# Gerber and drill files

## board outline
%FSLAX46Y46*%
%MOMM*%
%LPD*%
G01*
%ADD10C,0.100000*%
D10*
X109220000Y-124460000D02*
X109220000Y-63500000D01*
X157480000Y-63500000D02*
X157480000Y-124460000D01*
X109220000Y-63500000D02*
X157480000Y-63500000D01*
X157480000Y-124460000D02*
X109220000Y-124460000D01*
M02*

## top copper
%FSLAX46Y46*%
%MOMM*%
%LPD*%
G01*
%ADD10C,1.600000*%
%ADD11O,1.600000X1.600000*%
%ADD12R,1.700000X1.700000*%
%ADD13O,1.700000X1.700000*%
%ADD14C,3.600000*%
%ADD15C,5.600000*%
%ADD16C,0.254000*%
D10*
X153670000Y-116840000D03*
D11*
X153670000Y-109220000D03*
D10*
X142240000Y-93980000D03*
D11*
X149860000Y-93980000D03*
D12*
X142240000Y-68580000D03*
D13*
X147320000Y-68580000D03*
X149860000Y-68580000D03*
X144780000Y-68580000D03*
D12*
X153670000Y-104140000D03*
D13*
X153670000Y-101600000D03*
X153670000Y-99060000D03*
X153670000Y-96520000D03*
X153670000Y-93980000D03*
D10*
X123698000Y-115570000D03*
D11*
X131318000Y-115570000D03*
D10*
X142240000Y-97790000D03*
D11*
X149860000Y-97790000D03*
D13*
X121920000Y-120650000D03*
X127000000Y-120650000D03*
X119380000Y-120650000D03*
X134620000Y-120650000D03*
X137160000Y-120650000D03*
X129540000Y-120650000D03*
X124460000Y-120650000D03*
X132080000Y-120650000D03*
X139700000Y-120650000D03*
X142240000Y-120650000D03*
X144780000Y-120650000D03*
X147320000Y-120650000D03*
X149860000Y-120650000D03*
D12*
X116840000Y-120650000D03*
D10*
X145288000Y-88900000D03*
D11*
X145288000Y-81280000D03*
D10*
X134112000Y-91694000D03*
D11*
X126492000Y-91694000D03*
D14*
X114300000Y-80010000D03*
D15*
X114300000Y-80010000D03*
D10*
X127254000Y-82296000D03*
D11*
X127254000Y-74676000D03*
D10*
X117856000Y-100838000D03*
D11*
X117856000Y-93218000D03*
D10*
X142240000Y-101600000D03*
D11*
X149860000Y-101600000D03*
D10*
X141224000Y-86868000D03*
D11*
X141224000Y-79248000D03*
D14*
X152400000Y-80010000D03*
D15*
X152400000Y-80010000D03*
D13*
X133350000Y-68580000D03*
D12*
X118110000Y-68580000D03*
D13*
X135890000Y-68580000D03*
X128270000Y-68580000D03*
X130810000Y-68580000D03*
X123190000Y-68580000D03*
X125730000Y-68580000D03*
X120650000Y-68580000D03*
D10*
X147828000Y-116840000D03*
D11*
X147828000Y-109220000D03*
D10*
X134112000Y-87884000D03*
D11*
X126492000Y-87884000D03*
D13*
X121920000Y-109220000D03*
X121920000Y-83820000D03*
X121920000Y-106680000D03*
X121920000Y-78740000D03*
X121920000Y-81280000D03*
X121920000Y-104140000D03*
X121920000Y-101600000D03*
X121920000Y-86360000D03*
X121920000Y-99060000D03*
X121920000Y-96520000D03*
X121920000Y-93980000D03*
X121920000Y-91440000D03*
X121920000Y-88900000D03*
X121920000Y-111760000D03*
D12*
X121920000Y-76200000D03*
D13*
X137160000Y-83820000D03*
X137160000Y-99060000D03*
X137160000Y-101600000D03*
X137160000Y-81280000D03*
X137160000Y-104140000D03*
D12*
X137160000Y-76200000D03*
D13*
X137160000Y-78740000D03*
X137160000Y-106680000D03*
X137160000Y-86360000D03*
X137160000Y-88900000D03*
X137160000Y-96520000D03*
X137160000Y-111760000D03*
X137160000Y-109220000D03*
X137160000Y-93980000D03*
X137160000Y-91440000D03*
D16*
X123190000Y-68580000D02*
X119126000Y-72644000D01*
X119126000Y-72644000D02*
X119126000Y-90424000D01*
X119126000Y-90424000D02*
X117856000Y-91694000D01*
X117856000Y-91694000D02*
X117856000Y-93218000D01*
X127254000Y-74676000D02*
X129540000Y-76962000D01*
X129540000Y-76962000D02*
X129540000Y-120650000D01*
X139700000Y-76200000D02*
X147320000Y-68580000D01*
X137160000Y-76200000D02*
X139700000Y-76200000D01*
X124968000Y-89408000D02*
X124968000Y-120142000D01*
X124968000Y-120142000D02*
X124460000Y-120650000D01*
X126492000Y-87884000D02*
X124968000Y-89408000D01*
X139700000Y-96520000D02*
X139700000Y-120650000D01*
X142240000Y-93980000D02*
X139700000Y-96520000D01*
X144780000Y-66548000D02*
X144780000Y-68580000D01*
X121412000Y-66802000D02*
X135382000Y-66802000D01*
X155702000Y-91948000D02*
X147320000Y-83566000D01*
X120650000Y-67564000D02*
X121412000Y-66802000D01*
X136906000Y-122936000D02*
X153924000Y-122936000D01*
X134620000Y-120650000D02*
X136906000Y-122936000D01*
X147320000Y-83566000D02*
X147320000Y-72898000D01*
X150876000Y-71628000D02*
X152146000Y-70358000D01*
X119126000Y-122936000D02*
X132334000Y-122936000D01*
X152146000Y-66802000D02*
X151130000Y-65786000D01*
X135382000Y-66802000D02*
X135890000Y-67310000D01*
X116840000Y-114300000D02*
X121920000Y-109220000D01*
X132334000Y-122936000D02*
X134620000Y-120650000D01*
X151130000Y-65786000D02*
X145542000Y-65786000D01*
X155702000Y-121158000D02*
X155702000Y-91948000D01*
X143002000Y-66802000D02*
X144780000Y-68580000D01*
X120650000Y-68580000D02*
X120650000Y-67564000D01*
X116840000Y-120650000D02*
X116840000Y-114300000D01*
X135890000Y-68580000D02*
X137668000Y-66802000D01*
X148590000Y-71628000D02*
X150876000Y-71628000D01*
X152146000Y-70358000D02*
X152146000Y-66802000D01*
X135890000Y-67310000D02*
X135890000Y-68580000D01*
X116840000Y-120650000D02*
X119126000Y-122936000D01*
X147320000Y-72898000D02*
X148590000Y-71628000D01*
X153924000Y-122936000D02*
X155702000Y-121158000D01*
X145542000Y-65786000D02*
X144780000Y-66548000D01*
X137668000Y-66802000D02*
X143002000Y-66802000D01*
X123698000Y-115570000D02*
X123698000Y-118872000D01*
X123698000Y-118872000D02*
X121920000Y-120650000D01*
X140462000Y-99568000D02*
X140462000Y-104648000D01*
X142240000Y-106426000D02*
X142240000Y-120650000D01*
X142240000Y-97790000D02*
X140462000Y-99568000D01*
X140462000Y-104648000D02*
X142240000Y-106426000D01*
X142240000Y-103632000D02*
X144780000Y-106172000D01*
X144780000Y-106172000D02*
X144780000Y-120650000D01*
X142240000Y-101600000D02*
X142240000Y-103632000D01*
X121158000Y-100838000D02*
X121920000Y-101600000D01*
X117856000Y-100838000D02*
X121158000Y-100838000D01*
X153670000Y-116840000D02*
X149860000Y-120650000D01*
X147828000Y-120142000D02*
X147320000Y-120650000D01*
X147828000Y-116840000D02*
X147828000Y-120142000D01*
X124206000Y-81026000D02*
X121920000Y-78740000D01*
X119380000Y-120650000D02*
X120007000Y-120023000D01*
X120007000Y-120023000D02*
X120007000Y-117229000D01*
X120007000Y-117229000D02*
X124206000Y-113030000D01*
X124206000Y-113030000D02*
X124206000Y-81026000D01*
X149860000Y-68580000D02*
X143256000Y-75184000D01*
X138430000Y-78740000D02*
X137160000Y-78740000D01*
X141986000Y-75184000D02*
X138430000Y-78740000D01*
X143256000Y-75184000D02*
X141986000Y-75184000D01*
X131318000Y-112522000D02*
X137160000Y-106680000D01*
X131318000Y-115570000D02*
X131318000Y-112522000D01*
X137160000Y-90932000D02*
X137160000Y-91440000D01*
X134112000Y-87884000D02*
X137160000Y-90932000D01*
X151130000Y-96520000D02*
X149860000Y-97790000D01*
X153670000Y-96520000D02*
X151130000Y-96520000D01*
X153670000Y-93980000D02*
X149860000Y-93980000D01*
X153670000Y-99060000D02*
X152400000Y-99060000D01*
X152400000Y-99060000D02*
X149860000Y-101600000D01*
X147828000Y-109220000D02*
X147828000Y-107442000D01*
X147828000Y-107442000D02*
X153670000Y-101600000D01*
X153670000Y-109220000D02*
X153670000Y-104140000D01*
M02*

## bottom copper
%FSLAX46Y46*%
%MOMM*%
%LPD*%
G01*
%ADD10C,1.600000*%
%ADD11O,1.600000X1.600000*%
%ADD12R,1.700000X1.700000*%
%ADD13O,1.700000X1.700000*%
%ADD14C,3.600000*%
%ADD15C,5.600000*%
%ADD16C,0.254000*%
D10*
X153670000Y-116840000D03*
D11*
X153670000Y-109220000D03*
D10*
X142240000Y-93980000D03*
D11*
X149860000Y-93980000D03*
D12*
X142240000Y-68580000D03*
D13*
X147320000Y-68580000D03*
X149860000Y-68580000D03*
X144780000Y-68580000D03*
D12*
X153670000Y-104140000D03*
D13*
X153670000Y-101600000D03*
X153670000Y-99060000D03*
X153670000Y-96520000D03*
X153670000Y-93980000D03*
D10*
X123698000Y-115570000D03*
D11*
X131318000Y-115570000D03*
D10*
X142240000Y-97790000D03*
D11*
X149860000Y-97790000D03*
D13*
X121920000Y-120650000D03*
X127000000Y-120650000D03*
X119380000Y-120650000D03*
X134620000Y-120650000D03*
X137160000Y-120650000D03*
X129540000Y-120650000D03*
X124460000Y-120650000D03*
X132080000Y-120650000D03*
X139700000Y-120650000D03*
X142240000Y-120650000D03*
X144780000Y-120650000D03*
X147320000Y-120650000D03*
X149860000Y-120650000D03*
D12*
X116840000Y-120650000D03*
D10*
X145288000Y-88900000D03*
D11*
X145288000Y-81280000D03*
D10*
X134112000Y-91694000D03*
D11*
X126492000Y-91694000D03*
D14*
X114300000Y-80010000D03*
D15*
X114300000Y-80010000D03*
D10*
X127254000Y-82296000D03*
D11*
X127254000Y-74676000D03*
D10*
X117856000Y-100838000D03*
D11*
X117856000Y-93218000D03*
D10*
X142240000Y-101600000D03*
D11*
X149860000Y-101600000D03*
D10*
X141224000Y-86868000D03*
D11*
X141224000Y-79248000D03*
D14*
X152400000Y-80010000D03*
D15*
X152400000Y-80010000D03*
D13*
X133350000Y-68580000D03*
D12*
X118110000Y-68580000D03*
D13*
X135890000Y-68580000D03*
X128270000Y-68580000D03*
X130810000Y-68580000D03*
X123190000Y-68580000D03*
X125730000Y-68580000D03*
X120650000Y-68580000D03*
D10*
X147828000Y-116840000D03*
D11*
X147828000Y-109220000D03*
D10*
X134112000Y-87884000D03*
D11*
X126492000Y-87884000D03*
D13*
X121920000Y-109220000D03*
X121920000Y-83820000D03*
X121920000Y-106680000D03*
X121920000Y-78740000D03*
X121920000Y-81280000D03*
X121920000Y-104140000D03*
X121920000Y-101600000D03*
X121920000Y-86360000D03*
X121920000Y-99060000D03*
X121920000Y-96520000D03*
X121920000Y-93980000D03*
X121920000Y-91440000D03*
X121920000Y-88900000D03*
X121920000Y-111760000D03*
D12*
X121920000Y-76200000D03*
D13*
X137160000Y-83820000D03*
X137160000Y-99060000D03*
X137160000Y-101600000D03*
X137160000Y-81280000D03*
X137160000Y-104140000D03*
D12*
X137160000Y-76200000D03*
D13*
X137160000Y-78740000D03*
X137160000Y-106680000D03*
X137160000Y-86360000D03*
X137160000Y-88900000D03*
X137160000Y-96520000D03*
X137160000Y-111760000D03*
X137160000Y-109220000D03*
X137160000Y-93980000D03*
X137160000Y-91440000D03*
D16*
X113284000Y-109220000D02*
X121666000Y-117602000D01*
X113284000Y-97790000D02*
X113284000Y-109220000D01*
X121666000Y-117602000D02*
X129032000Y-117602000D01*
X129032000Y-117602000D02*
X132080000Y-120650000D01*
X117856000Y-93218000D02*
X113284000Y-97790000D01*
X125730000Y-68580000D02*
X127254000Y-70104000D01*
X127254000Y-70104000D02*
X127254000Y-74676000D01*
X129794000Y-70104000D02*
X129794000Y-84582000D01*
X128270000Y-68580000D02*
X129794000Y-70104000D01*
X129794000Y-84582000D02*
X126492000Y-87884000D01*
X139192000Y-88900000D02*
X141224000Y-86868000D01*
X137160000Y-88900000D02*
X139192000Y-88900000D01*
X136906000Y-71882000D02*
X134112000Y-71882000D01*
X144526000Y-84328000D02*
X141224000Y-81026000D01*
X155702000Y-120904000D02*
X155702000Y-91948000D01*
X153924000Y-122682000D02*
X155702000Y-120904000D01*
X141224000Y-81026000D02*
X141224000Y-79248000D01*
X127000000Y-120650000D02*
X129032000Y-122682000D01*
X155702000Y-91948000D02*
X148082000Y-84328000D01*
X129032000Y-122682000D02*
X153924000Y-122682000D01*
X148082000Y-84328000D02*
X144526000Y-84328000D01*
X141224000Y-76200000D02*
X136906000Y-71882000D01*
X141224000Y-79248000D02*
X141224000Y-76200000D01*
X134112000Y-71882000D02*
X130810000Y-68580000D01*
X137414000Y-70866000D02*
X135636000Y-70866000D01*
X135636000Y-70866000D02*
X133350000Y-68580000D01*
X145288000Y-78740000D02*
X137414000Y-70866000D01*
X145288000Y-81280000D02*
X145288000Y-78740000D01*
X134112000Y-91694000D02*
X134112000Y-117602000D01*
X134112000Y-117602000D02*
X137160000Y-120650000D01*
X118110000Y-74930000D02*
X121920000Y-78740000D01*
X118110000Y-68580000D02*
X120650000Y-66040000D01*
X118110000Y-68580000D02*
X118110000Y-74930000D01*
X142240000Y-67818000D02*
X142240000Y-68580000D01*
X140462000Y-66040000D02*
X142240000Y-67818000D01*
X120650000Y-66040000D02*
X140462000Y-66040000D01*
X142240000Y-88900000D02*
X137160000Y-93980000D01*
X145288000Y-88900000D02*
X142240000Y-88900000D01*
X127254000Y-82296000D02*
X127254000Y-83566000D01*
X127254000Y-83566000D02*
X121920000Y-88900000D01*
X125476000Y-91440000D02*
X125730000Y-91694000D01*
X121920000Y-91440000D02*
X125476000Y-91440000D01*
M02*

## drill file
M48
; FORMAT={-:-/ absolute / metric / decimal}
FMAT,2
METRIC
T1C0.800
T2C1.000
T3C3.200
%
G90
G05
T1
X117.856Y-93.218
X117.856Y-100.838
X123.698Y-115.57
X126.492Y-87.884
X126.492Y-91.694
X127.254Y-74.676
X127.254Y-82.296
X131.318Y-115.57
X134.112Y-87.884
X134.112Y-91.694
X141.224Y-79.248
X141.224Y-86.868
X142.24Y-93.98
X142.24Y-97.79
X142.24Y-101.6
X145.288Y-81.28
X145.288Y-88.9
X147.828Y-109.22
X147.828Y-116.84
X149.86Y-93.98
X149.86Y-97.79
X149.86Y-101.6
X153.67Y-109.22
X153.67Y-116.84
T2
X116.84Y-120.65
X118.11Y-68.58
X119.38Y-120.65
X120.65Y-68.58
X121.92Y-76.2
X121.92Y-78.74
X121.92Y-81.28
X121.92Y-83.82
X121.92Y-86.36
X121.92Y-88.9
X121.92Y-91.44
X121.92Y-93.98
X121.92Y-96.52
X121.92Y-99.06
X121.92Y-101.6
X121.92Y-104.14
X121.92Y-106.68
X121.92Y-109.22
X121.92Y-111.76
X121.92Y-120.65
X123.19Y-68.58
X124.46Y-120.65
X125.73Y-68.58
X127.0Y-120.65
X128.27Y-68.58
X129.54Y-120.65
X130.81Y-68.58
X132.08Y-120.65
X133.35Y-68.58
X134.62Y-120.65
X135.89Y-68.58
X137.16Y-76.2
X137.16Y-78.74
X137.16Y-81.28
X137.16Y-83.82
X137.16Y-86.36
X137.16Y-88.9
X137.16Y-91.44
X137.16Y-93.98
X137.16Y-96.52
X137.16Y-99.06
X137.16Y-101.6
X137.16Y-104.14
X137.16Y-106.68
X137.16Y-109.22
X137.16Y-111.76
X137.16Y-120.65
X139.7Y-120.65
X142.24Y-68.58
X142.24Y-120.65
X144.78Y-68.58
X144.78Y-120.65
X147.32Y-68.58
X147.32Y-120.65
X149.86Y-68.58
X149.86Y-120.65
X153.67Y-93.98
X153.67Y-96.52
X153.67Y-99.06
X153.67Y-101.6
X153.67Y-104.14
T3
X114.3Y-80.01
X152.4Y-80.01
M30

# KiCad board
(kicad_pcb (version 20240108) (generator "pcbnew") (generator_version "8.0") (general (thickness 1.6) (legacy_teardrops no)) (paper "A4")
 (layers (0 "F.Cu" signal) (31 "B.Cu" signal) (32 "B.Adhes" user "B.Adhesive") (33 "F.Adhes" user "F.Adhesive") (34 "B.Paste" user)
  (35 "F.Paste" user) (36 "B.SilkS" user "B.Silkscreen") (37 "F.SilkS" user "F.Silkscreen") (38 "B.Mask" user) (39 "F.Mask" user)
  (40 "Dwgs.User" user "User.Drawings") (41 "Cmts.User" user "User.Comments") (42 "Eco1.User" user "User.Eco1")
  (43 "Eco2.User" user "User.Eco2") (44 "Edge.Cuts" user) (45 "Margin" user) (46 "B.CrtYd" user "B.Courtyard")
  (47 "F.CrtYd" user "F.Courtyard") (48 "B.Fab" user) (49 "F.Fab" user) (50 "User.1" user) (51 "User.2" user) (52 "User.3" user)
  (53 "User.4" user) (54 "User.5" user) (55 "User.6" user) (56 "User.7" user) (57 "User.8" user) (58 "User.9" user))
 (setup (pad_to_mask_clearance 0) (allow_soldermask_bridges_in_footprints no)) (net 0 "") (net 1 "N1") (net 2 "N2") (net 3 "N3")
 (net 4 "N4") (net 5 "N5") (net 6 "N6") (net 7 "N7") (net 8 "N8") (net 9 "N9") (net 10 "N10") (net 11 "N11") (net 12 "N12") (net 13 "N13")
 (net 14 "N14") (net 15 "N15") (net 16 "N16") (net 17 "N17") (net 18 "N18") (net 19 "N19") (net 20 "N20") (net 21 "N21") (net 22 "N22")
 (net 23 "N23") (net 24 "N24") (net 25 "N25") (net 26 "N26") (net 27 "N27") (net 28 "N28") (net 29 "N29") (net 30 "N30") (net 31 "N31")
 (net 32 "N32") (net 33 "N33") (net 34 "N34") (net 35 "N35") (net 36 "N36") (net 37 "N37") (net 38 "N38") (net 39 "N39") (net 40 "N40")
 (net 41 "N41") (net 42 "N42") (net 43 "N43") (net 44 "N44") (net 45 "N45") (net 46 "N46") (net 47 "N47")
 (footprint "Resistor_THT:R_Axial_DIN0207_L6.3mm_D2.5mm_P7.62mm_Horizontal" (layer "F.Cu") (at 153.67 116.84 90)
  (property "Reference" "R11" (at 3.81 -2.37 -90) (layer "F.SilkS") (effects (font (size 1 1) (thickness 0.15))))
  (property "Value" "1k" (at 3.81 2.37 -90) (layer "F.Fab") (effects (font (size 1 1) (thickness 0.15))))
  (pad "1" thru_hole circle (at 0 0 90) (size 1.6 1.6) (drill 0.8) (layers "*.Cu" "*.Mask") (remove_unused_layers no) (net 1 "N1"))
  (pad "2" thru_hole oval (at 7.62 0 90) (size 1.6 1.6) (drill 0.8) (layers "*.Cu" "*.Mask") (remove_unused_layers no) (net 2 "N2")))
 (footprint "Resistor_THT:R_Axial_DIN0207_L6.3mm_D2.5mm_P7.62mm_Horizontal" (layer "F.Cu") (at 142.24 93.98)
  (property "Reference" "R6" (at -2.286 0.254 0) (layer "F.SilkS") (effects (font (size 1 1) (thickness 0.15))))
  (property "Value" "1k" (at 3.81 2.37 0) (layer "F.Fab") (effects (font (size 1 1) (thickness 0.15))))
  (pad "1" thru_hole circle (at 0 0) (size 1.6 1.6) (drill 0.8) (layers "*.Cu" "*.Mask") (remove_unused_layers no) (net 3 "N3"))
  (pad "2" thru_hole oval (at 7.62 0) (size 1.6 1.6) (drill 0.8) (layers "*.Cu" "*.Mask") (remove_unused_layers no) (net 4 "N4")))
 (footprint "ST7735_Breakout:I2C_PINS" (layer "F.Cu") (at 142.24 68.58 90)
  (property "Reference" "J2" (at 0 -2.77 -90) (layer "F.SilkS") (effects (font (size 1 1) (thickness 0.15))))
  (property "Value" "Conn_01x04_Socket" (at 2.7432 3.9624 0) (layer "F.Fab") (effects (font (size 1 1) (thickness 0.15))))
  (pad "GND" thru_hole rect (at 0 0 180) (size 1.7 1.7) (drill 1) (layers "*.Cu" "*.Mask") (remove_unused_layers no) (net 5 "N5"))
  (pad "SCK" thru_hole oval (at 0 5.08 90) (size 1.7 1.7) (drill 1) (layers "*.Cu" "*.Mask") (remove_unused_layers no) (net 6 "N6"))
  (pad "SDA" thru_hole oval (at 0 7.62 90) (size 1.7 1.7) (drill 1) (layers "*.Cu" "*.Mask") (remove_unused_layers no) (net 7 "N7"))
  (pad "VCC" thru_hole oval (at 0 2.54 90) (size 1.7 1.7) (drill 1) (layers "*.Cu" "*.Mask") (remove_unused_layers no) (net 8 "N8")))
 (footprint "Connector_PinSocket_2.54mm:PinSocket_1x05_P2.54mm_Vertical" (layer "F.Cu") (at 153.67 104.14 180)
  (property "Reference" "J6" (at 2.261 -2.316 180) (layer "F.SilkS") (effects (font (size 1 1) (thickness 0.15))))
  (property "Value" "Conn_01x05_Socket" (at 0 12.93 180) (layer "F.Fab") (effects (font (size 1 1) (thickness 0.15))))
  (pad "1" thru_hole rect (at 0 0 180) (size 1.7 1.7) (drill 1) (layers "*.Cu" "*.Mask") (remove_unused_layers no) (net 2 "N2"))
  (pad "2" thru_hole oval (at 0 2.54 180) (size 1.7 1.7) (drill 1) (layers "*.Cu" "*.Mask") (remove_unused_layers no) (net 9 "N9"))
  (pad "3" thru_hole oval (at 0 5.08 180) (size 1.7 1.7) (drill 1) (layers "*.Cu" "*.Mask") (remove_unused_layers no) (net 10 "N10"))
  (pad "4" thru_hole oval (at 0 7.62 180) (size 1.7 1.7) (drill 1) (layers "*.Cu" "*.Mask") (remove_unused_layers no) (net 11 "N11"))
  (pad "5" thru_hole oval (at 0 10.16 180) (size 1.7 1.7) (drill 1) (layers "*.Cu" "*.Mask") (remove_unused_layers no) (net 4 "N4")))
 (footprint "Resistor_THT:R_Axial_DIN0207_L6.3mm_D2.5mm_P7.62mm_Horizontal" (layer "F.Cu") (at 123.698 115.57)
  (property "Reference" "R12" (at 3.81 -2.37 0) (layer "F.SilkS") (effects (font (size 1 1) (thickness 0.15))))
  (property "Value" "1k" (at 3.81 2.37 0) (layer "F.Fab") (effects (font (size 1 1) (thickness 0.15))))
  (pad "1" thru_hole circle (at 0 0) (size 1.6 1.6) (drill 0.8) (layers "*.Cu" "*.Mask") (remove_unused_layers no) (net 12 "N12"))
  (pad "2" thru_hole oval (at 7.62 0) (size 1.6 1.6) (drill 0.8) (layers "*.Cu" "*.Mask") (remove_unused_layers no) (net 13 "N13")))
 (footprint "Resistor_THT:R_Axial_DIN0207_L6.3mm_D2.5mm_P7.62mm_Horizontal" (layer "F.Cu") (at 142.24 97.79)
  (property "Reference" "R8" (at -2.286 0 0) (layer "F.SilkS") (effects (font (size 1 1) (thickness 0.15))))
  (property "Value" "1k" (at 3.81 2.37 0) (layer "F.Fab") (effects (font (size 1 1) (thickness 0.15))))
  (pad "1" thru_hole circle (at 0 0) (size 1.6 1.6) (drill 0.8) (layers "*.Cu" "*.Mask") (remove_unused_layers no) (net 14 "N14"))
  (pad "2" thru_hole oval (at 7.62 0) (size 1.6 1.6) (drill 0.8) (layers "*.Cu" "*.Mask") (remove_unused_layers no) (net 11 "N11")))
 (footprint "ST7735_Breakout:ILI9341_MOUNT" (layer "F.Cu") (at 116.84 120.65 90)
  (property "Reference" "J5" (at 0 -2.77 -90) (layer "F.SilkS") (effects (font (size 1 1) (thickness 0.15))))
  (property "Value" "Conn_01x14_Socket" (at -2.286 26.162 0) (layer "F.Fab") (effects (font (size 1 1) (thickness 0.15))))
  (pad "CS" thru_hole oval (at 0 5.08 90) (size 1.7 1.7) (drill 1) (layers "*.Cu" "*.Mask") (remove_unused_layers no) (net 12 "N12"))
  (pad "DC" thru_hole oval (at 0 10.16 90) (size 1.7 1.7) (drill 1) (layers "*.Cu" "*.Mask") (remove_unused_layers no) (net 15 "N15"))
  (pad "GND" thru_hole oval (at 0 2.54 90) (size 1.7 1.7) (drill 1) (layers "*.Cu" "*.Mask") (remove_unused_layers no) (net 5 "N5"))
  (pad "LED" thru_hole oval (at 0 17.78 90) (size 1.7 1.7) (drill 1) (layers "*.Cu" "*.Mask") (remove_unused_layers no) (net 8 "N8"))
  (pad "MISO" thru_hole oval (at 0 20.32 90) (size 1.7 1.7) (drill 1) (layers "*.Cu" "*.Mask") (remove_unused_layers no) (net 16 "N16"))
  (pad "MOSI" thru_hole oval (at 0 12.7 180) (size 1.7 1.7) (drill 1) (layers "*.Cu" "*.Mask") (remove_unused_layers no) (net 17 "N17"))
  (pad "RESET" thru_hole oval (at 0 7.62 90) (size 1.7 1.7) (drill 1) (layers "*.Cu" "*.Mask") (remove_unused_layers no) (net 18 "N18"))
  (pad "SCK" thru_hole oval (at 0 15.24 90) (size 1.7 1.7) (drill 1) (layers "*.Cu" "*.Mask") (remove_unused_layers no) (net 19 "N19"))
  (pad "T_CLK" thru_hole oval (at 0 22.86 90) (size 1.7 1.7) (drill 1) (layers "*.Cu" "*.Mask") (remove_unused_layers no) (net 3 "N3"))
  (pad "T_CS" thru_hole oval (at 0 25.4 90) (size 1.7 1.7) (drill 1) (layers "*.Cu" "*.Mask") (remove_unused_layers no) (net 14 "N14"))
  (pad "T_DIN" thru_hole oval (at 0 27.94 90) (size 1.7 1.7) (drill 1) (layers "*.Cu" "*.Mask") (remove_unused_layers no) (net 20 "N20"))
  (pad "T_DO" thru_hole oval (at 0 30.48 90) (size 1.7 1.7) (drill 1) (layers "*.Cu" "*.Mask") (remove_unused_layers no) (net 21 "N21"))
  (pad "T_IRQ" thru_hole oval (at 0 33.02 90) (size 1.7 1.7) (drill 1) (layers "*.Cu" "*.Mask") (remove_unused_layers no) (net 1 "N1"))
  (pad "VCC" thru_hole rect (at 0 0 90) (size 1.7 1.7) (drill 1) (layers "*.Cu" "*.Mask") (remove_unused_layers no) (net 8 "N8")))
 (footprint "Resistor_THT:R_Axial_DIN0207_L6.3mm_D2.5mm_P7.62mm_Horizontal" (layer "F.Cu") (at 145.288 88.9 90)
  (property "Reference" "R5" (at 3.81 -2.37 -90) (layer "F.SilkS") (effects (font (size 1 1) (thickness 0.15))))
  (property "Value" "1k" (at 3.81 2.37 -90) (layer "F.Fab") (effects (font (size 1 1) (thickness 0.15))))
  (pad "1" thru_hole circle (at 0 0 90) (size 1.6 1.6) (drill 0.8) (layers "*.Cu" "*.Mask") (remove_unused_layers no) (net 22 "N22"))
  (pad "2" thru_hole oval (at 7.62 0 90) (size 1.6 1.6) (drill 0.8) (layers "*.Cu" "*.Mask") (remove_unused_layers no) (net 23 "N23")))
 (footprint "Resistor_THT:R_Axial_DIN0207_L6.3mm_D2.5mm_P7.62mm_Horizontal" (layer "F.Cu") (at 134.112 91.694 180)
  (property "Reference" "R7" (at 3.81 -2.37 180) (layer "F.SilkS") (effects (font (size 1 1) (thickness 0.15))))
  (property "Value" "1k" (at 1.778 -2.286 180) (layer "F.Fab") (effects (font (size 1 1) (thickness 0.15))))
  (pad "1" thru_hole circle (at 0 0 180) (size 1.6 1.6) (drill 0.8) (layers "*.Cu" "*.Mask") (remove_unused_layers no) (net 16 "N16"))
  (pad "2" thru_hole oval (at 7.62 0 180) (size 1.6 1.6) (drill 0.8) (layers "*.Cu" "*.Mask") (remove_unused_layers no) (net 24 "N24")))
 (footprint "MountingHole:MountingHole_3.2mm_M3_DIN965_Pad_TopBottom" (layer "F.Cu") (at 114.3 80.01)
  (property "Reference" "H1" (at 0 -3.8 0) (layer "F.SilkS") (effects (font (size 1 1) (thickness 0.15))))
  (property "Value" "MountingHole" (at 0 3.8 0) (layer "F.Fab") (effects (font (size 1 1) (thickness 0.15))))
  (pad "1" thru_hole circle (at 0 0) (size 3.6 3.6) (drill 3.2) (layers "*.Cu" "*.Mask") (remove_unused_layers no))
  (pad "1" connect circle (at 0 0) (size 5.6 5.6) (layers "F.Cu" "F.Mask"))
  (pad "1" connect circle (at 0 0) (size 5.6 5.6) (layers "B.Cu" "B.Mask")))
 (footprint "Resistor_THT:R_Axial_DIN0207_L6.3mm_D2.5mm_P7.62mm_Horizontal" (layer "F.Cu") (at 127.254 82.296 90)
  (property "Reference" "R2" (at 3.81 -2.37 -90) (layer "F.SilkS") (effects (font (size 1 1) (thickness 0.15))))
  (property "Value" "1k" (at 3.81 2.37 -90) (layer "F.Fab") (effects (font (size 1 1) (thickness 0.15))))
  (pad "1" thru_hole circle (at 0 0 90) (size 1.6 1.6) (drill 0.8) (layers "*.Cu" "*.Mask") (remove_unused_layers no) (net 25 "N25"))
  (pad "2" thru_hole oval (at 7.62 0 90) (size 1.6 1.6) (drill 0.8) (layers "*.Cu" "*.Mask") (remove_unused_layers no) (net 17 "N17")))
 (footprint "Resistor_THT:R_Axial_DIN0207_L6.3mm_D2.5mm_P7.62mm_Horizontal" (layer "F.Cu") (at 117.856 100.838 90)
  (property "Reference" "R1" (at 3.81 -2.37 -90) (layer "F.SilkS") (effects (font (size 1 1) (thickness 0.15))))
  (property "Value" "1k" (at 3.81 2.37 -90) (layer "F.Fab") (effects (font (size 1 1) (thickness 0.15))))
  (pad "1" thru_hole circle (at 0 0 90) (size 1.6 1.6) (drill 0.8) (layers "*.Cu" "*.Mask") (remove_unused_layers no) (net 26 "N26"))
  (pad "2" thru_hole oval (at 7.62 0 90) (size 1.6 1.6) (drill 0.8) (layers "*.Cu" "*.Mask") (remove_unused_layers no) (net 19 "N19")))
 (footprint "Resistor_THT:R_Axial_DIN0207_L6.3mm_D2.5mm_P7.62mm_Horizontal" (layer "F.Cu") (at 142.24 101.6)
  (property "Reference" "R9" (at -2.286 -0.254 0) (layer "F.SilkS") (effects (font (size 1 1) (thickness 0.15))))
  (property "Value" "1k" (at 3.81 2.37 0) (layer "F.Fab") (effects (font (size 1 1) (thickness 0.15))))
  (pad "1" thru_hole circle (at 0 0) (size 1.6 1.6) (drill 0.8) (layers "*.Cu" "*.Mask") (remove_unused_layers no) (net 20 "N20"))
  (pad "2" thru_hole oval (at 7.62 0) (size 1.6 1.6) (drill 0.8) (layers "*.Cu" "*.Mask") (remove_unused_layers no) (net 10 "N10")))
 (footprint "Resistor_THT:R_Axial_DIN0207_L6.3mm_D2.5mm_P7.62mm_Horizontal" (layer "F.Cu") (at 141.224 86.868 90)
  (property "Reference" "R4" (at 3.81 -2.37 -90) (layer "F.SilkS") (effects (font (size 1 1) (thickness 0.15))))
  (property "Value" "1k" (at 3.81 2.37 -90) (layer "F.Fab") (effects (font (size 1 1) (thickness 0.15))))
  (pad "1" thru_hole circle (at 0 0 90) (size 1.6 1.6) (drill 0.8) (layers "*.Cu" "*.Mask") (remove_unused_layers no) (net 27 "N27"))
  (pad "2" thru_hole oval (at 7.62 0 90) (size 1.6 1.6) (drill 0.8) (layers "*.Cu" "*.Mask") (remove_unused_layers no) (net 15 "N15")))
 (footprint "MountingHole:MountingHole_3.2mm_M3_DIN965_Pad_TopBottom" (layer "F.Cu") (at 152.4 80.01)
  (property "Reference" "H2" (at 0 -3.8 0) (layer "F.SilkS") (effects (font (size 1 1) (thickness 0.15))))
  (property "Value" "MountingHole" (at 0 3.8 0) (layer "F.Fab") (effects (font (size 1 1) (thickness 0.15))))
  (pad "1" thru_hole circle (at 0 0) (size 3.6 3.6) (drill 3.2) (layers "*.Cu" "*.Mask") (remove_unused_layers no))
  (pad "1" connect circle (at 0 0) (size 5.6 5.6) (layers "F.Cu" "F.Mask"))
  (pad "1" connect circle (at 0 0) (size 5.6 5.6) (layers "B.Cu" "B.Mask")))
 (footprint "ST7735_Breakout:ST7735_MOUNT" (layer "F.Cu") (at 118.11 68.58 90)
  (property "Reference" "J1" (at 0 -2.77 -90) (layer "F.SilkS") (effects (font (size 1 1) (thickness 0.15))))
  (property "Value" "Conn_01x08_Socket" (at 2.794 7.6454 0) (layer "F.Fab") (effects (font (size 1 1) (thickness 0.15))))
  (pad "CS" thru_hole oval (at 0 15.24 90) (size 1.7 1.7) (drill 1) (layers "*.Cu" "*.Mask") (remove_unused_layers no) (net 23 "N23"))
  (pad "GND" thru_hole rect (at 0 0 90) (size 1.7 1.7) (drill 1) (layers "*.Cu" "*.Mask") (remove_unused_layers no) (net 5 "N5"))
  (pad "LEDA" thru_hole oval (at 0 17.78 90) (size 1.7 1.7) (drill 1) (layers "*.Cu" "*.Mask") (remove_unused_layers no) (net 8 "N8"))
  (pad "RES" thru_hole oval (at 0 10.16 90) (size 1.7 1.7) (drill 1) (layers "*.Cu" "*.Mask") (remove_unused_layers no) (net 18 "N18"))
  (pad "RS_DC" thru_hole oval (at 0 12.7 90) (size 1.7 1.7) (drill 1) (layers "*.Cu" "*.Mask") (remove_unused_layers no) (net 15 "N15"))
  (pad "SCK" thru_hole oval (at 0 5.08 90) (size 1.7 1.7) (drill 1) (layers "*.Cu" "*.Mask") (remove_unused_layers no) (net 19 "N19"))
  (pad "SDA" thru_hole oval (at 0 7.62 90) (size 1.7 1.7) (drill 1) (layers "*.Cu" "*.Mask") (remove_unused_layers no) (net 17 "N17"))
  (pad "VCC" thru_hole oval (at 0 2.54 90) (size 1.7 1.7) (drill 1) (layers "*.Cu" "*.Mask") (remove_unused_layers no) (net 8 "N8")))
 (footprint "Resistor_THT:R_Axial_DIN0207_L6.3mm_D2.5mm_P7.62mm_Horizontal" (layer "F.Cu") (at 147.828 116.84 90)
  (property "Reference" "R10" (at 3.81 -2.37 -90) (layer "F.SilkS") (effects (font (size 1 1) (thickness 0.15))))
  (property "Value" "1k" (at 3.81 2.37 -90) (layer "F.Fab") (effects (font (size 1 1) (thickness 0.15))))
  (pad "1" thru_hole circle (at 0 0 90) (size 1.6 1.6) (drill 0.8) (layers "*.Cu" "*.Mask") (remove_unused_layers no) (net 21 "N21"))
  (pad "2" thru_hole oval (at 7.62 0 90) (size 1.6 1.6) (drill 0.8) (layers "*.Cu" "*.Mask") (remove_unused_layers no) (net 9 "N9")))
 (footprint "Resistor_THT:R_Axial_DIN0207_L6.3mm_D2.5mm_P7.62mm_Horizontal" (layer "F.Cu") (at 134.112 87.884 180)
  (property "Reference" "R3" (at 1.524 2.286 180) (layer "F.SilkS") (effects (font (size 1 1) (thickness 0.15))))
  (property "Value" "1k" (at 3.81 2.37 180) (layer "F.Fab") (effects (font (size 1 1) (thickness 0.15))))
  (pad "1" thru_hole circle (at 0 0 180) (size 1.6 1.6) (drill 0.8) (layers "*.Cu" "*.Mask") (remove_unused_layers no) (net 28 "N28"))
  (pad "2" thru_hole oval (at 7.62 0 180) (size 1.6 1.6) (drill 0.8) (layers "*.Cu" "*.Mask") (remove_unused_layers no) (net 18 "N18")))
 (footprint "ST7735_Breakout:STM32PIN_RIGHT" (layer "B.Cu") (at 121.92 76.2 180)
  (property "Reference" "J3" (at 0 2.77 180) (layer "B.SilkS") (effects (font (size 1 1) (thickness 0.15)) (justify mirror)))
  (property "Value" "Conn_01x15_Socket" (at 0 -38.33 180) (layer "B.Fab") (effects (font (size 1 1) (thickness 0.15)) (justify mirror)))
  (pad "3V3" thru_hole oval (at 0 -33.02 180) (size 1.7 1.7) (drill 1) (layers "*.Cu" "*.Mask") (remove_unused_layers no) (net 8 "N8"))
  (pad "5V" thru_hole oval (at 0 -7.62 180) (size 1.7 1.7) (drill 1) (layers "*.Cu" "*.Mask") (remove_unused_layers no) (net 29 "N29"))
  (pad "AREF" thru_hole oval (at 0 -30.48 180) (size 1.7 1.7) (drill 1) (layers "*.Cu" "*.Mask") (remove_unused_layers no) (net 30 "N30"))
  (pad "GND" thru_hole oval (at 0 -2.54 180) (size 1.7 1.7) (drill 1) (layers "*.Cu" "*.Mask") (remove_unused_layers no) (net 5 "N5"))
  (pad "NRST" thru_hole oval (at 0 -5.08 180) (size 1.7 1.7) (drill 1) (layers "*.Cu" "*.Mask") (remove_unused_layers no) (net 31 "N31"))
  (pad "PA0" thru_hole oval (at 0 -27.94 180) (size 1.7 1.7) (drill 1) (layers "*.Cu" "*.Mask") (remove_unused_layers no) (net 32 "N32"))
  (pad "PA1" thru_hole oval (at 0 -25.4 180) (size 1.7 1.7) (drill 1) (layers "*.Cu" "*.Mask") (remove_unused_layers no) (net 26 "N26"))
  (pad "PA2" thru_hole oval (at 0 -10.16 180) (size 1.7 1.7) (drill 1) (layers "*.Cu" "*.Mask") (remove_unused_layers no) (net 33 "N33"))
  (pad "PA3" thru_hole oval (at 0 -22.86 180) (size 1.7 1.7) (drill 1) (layers "*.Cu" "*.Mask") (remove_unused_layers no) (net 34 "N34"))
  (pad "PA4" thru_hole oval (at 0 -20.32 180) (size 1.7 1.7) (drill 1) (layers "*.Cu" "*.Mask") (remove_unused_layers no) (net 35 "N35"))
  (pad "PA5" thru_hole oval (at 0 -17.78 180) (size 1.7 1.7) (drill 1) (layers "*.Cu" "*.Mask") (remove_unused_layers no) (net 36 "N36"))
  (pad "PA6" thru_hole oval (at 0 -15.24 180) (size 1.7 1.7) (drill 1) (layers "*.Cu" "*.Mask") (remove_unused_layers no) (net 24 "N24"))
  (pad "PA7" thru_hole oval (at 0 -12.7 180) (size 1.7 1.7) (drill 1) (layers "*.Cu" "*.Mask") (remove_unused_layers no) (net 25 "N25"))
  (pad "PB3" thru_hole oval (at 0 -35.56 90) (size 1.7 1.7) (drill 1) (layers "*.Cu" "*.Mask") (remove_unused_layers no) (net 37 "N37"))
  (pad "VIN" thru_hole rect (at 0 0 180) (size 1.7 1.7) (drill 1) (layers "*.Cu" "*.Mask") (remove_unused_layers no) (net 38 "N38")))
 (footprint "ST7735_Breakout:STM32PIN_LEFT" (layer "B.Cu") (at 137.16 76.2 180)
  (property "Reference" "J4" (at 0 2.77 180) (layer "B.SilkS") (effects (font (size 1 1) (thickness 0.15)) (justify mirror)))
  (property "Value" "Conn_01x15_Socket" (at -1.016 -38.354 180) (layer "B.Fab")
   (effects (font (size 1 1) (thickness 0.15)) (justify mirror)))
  (pad "GND" thru_hole oval (at 0 -7.62 180) (size 1.7 1.7) (drill 1) (layers "*.Cu" "*.Mask") (remove_unused_layers no) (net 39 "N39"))
  (pad "NC1" thru_hole oval (at 0 -22.86 180) (size 1.7 1.7) (drill 1) (layers "*.Cu" "*.Mask") (remove_unused_layers no) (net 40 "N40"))
  (pad "NC2" thru_hole oval (at 0 -25.4 180) (size 1.7 1.7) (drill 1) (layers "*.Cu" "*.Mask") (remove_unused_layers no) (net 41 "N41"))
  (pad "NRST" thru_hole oval (at 0 -5.08 180) (size 1.7 1.7) (drill 1) (layers "*.Cu" "*.Mask") (remove_unused_layers no) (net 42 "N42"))
  (pad "PA8" thru_hole oval (at 0 -27.94 180) (size 1.7 1.7) (drill 1) (layers "*.Cu" "*.Mask") (remove_unused_layers no) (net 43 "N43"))
  (pad "PA9" thru_hole rect (at 0 0 90) (size 1.7 1.7) (drill 1) (layers "*.Cu" "*.Mask") (remove_unused_layers no) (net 6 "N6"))
  (pad "PA10" thru_hole oval (at 0 -2.54 180) (size 1.7 1.7) (drill 1) (layers "*.Cu" "*.Mask") (remove_unused_layers no) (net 7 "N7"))
  (pad "PA11" thru_hole oval (at 0 -30.48 180) (size 1.7 1.7) (drill 1) (layers "*.Cu" "*.Mask") (remove_unused_layers no) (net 13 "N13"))
  (pad "PA12" thru_hole oval (at 0 -10.16 180) (size 1.7 1.7) (drill 1) (layers "*.Cu" "*.Mask") (remove_unused_layers no) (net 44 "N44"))
  (pad "PB0" thru_hole oval (at 0 -12.7 180) (size 1.7 1.7) (drill 1) (layers "*.Cu" "*.Mask") (remove_unused_layers no) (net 27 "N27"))
  (pad "PB1" thru_hole oval (at 0 -20.32 180) (size 1.7 1.7) (drill 1) (layers "*.Cu" "*.Mask") (remove_unused_layers no) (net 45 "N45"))
  (pad "PB4" thru_hole oval (at 0 -35.56 90) (size 1.7 1.7) (drill 1) (layers "*.Cu" "*.Mask") (remove_unused_layers no) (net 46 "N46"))
  (pad "PB5" thru_hole oval (at 0 -33.02 180) (size 1.7 1.7) (drill 1) (layers "*.Cu" "*.Mask") (remove_unused_layers no) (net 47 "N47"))
  (pad "PB6" thru_hole oval (at 0 -17.78 180) (size 1.7 1.7) (drill 1) (layers "*.Cu" "*.Mask") (remove_unused_layers no) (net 22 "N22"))
  (pad "PB7" thru_hole oval (at 0 -15.24 180) (size 1.7 1.7) (drill 1) (layers "*.Cu" "*.Mask") (remove_unused_layers no) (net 28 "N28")))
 (gr_line (start 109.22 124.46) (end 109.22 63.5) (stroke (width 0.1) (type default)) (layer "Edge.Cuts"))
 (gr_line (start 157.48 63.5) (end 157.48 124.46) (stroke (width 0.1) (type default)) (layer "Edge.Cuts"))
 (gr_line (start 109.22 63.5) (end 157.48 63.5) (stroke (width 0.1) (type default)) (layer "Edge.Cuts"))
 (gr_line (start 157.48 124.46) (end 109.22 124.46) (stroke (width 0.1) (type default)) (layer "Edge.Cuts"))
 (segment (start 123.19 68.58) (end 119.126 72.644) (width 0.254) (layer "F.Cu") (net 19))
 (segment (start 119.126 72.644) (end 119.126 90.424) (width 0.254) (layer "F.Cu") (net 19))
 (segment (start 119.126 90.424) (end 117.856 91.694) (width 0.254) (layer "F.Cu") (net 19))
 (segment (start 117.856 91.694) (end 117.856 93.218) (width 0.254) (layer "F.Cu") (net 19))
 (segment (start 113.284 109.22) (end 121.666 117.602) (width 0.254) (layer "B.Cu") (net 19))
 (segment (start 113.284 97.79) (end 113.284 109.22) (width 0.254) (layer "B.Cu") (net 19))
 (segment (start 121.666 117.602) (end 129.032 117.602) (width 0.254) (layer "B.Cu") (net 19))
 (segment (start 129.032 117.602) (end 132.08 120.65) (width 0.254) (layer "B.Cu") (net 19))
 (segment (start 117.856 93.218) (end 113.284 97.79) (width 0.254) (layer "B.Cu") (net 19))
 (segment (start 127.254 74.676) (end 129.54 76.962) (width 0.254) (layer "F.Cu") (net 17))
 (segment (start 129.54 76.962) (end 129.54 120.65) (width 0.254) (layer "F.Cu") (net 17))
 (segment (start 125.73 68.58) (end 127.254 70.104) (width 0.254) (layer "B.Cu") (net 17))
 (segment (start 127.254 70.104) (end 127.254 74.676) (width 0.254) (layer "B.Cu") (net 17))
 (segment (start 139.7 76.2) (end 147.32 68.58) (width 0.254) (layer "F.Cu") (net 6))
 (segment (start 137.16 76.2) (end 139.7 76.2) (width 0.254) (layer "F.Cu") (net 6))
 (segment (start 124.968 89.408) (end 124.968 120.142) (width 0.254) (layer "F.Cu") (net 18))
 (segment (start 124.968 120.142) (end 124.46 120.65) (width 0.254) (layer "F.Cu") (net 18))
 (segment (start 126.492 87.884) (end 124.968 89.408) (width 0.254) (layer "F.Cu") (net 18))
 (segment (start 129.794 70.104) (end 129.794 84.582) (width 0.254) (layer "B.Cu") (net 18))
 (segment (start 128.27 68.58) (end 129.794 70.104) (width 0.254) (layer "B.Cu") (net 18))
 (segment (start 129.794 84.582) (end 126.492 87.884) (width 0.254) (layer "B.Cu") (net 18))
 (segment (start 139.192 88.9) (end 141.224 86.868) (width 0.254) (layer "B.Cu") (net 27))
 (segment (start 137.16 88.9) (end 139.192 88.9) (width 0.254) (layer "B.Cu") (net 27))
 (segment (start 136.906 71.882) (end 134.112 71.882) (width 0.254) (layer "B.Cu") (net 15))
 (segment (start 144.526 84.328) (end 141.224 81.026) (width 0.254) (layer "B.Cu") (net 15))
 (segment (start 155.702 120.904) (end 155.702 91.948) (width 0.254) (layer "B.Cu") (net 15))
 (segment (start 153.924 122.682) (end 155.702 120.904) (width 0.254) (layer "B.Cu") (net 15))
 (segment (start 141.224 81.026) (end 141.224 79.248) (width 0.254) (layer "B.Cu") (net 15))
 (segment (start 127 120.65) (end 129.032 122.682) (width 0.254) (layer "B.Cu") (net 15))
 (segment (start 155.702 91.948) (end 148.082 84.328) (width 0.254) (layer "B.Cu") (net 15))
 (segment (start 129.032 122.682) (end 153.924 122.682) (width 0.254) (layer "B.Cu") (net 15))
 (segment (start 148.082 84.328) (end 144.526 84.328) (width 0.254) (layer "B.Cu") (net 15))
 (segment (start 141.224 76.2) (end 136.906 71.882) (width 0.254) (layer "B.Cu") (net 15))
 (segment (start 141.224 79.248) (end 141.224 76.2) (width 0.254) (layer "B.Cu") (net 15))
 (segment (start 134.112 71.882) (end 130.81 68.58) (width 0.254) (layer "B.Cu") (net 15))
 (segment (start 137.414 70.866) (end 135.636 70.866) (width 0.254) (layer "B.Cu") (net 23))
 (segment (start 135.636 70.866) (end 133.35 68.58) (width 0.254) (layer "B.Cu") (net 23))
 (segment (start 145.288 78.74) (end 137.414 70.866) (width 0.254) (layer "B.Cu") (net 23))
 (segment (start 145.288 81.28) (end 145.288 78.74) (width 0.254) (layer "B.Cu") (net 23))
 (segment (start 139.7 96.52) (end 139.7 120.65) (width 0.254) (layer "F.Cu") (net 3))
 (segment (start 142.24 93.98) (end 139.7 96.52) (width 0.254) (layer "F.Cu") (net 3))
 (segment (start 134.112 91.694) (end 134.112 117.602) (width 0.254) (layer "B.Cu") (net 16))
 (segment (start 134.112 117.602) (end 137.16 120.65) (width 0.254) (layer "B.Cu") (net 16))
 (segment (start 144.78 66.548) (end 144.78 68.58) (width 0.254) (layer "F.Cu") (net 8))
 (segment (start 121.412 66.802) (end 135.382 66.802) (width 0.254) (layer "F.Cu") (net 8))
 (segment (start 155.702 91.948) (end 147.32 83.566) (width 0.254) (layer "F.Cu") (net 8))
 (segment (start 120.65 67.564) (end 121.412 66.802) (width 0.254) (layer "F.Cu") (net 8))
 (segment (start 136.906 122.936) (end 153.924 122.936) (width 0.254) (layer "F.Cu") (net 8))
 (segment (start 134.62 120.65) (end 136.906 122.936) (width 0.254) (layer "F.Cu") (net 8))
 (segment (start 147.32 83.566) (end 147.32 72.898) (width 0.254) (layer "F.Cu") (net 8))
 (segment (start 150.876 71.628) (end 152.146 70.358) (width 0.254) (layer "F.Cu") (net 8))
 (segment (start 119.126 122.936) (end 132.334 122.936) (width 0.254) (layer "F.Cu") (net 8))
 (segment (start 152.146 66.802) (end 151.13 65.786) (width 0.254) (layer "F.Cu") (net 8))
 (segment (start 135.382 66.802) (end 135.89 67.31) (width 0.254) (layer "F.Cu") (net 8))
 (segment (start 116.84 114.3) (end 121.92 109.22) (width 0.254) (layer "F.Cu") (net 8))
 (segment (start 132.334 122.936) (end 134.62 120.65) (width 0.254) (layer "F.Cu") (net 8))
 (segment (start 151.13 65.786) (end 145.542 65.786) (width 0.254) (layer "F.Cu") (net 8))
 (segment (start 155.702 121.158) (end 155.702 91.948) (width 0.254) (layer "F.Cu") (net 8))
 (segment (start 143.002 66.802) (end 144.78 68.58) (width 0.254) (layer "F.Cu") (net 8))
 (segment (start 120.65 68.58) (end 120.65 67.564) (width 0.254) (layer "F.Cu") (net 8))
 (segment (start 116.84 120.65) (end 116.84 114.3) (width 0.254) (layer "F.Cu") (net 8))
 (segment (start 135.89 68.58) (end 137.668 66.802) (width 0.254) (layer "F.Cu") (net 8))
 (segment (start 148.59 71.628) (end 150.876 71.628) (width 0.254) (layer "F.Cu") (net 8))
 (segment (start 152.146 70.358) (end 152.146 66.802) (width 0.254) (layer "F.Cu") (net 8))
 (segment (start 135.89 67.31) (end 135.89 68.58) (width 0.254) (layer "F.Cu") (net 8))
 (segment (start 116.84 120.65) (end 119.126 122.936) (width 0.254) (layer "F.Cu") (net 8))
 (segment (start 147.32 72.898) (end 148.59 71.628) (width 0.254) (layer "F.Cu") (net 8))
 (segment (start 153.924 122.936) (end 155.702 121.158) (width 0.254) (layer "F.Cu") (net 8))
 (segment (start 145.542 65.786) (end 144.78 66.548) (width 0.254) (layer "F.Cu") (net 8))
 (segment (start 137.668 66.802) (end 143.002 66.802) (width 0.254) (layer "F.Cu") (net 8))
 (segment (start 123.698 115.57) (end 123.698 118.872) (width 0.254) (layer "F.Cu") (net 12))
 (segment (start 123.698 118.872) (end 121.92 120.65) (width 0.254) (layer "F.Cu") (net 12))
 (segment (start 140.462 99.568) (end 140.462 104.648) (width 0.254) (layer "F.Cu") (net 14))
 (segment (start 142.24 106.426) (end 142.24 120.65) (width 0.254) (layer "F.Cu") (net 14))
 (segment (start 142.24 97.79) (end 140.462 99.568) (width 0.254) (layer "F.Cu") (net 14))
 (segment (start 140.462 104.648) (end 142.24 106.426) (width 0.254) (layer "F.Cu") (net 14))
 (segment (start 142.24 103.632) (end 144.78 106.172) (width 0.254) (layer "F.Cu") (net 20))
 (segment (start 144.78 106.172) (end 144.78 120.65) (width 0.254) (layer "F.Cu") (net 20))
 (segment (start 142.24 101.6) (end 142.24 103.632) (width 0.254) (layer "F.Cu") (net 20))
 (segment (start 121.158 100.838) (end 121.92 101.6) (width 0.254) (layer "F.Cu") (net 26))
 (segment (start 117.856 100.838) (end 121.158 100.838) (width 0.254) (layer "F.Cu") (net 26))
 (segment (start 153.67 116.84) (end 149.86 120.65) (width 0.254) (layer "F.Cu") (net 1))
 (segment (start 147.828 120.142) (end 147.32 120.65) (width 0.254) (layer "F.Cu") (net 21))
 (segment (start 147.828 116.84) (end 147.828 120.142) (width 0.254) (layer "F.Cu") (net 21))
 (segment (start 124.206 81.026) (end 121.92 78.74) (width 0.254) (layer "F.Cu") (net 5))
 (segment (start 119.38 120.65) (end 120.007 120.023) (width 0.254) (layer "F.Cu") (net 5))
 (segment (start 120.007 120.023) (end 120.007 117.229) (width 0.254) (layer "F.Cu") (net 5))
 (segment (start 120.007 117.229) (end 124.206 113.03) (width 0.254) (layer "F.Cu") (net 5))
 (segment (start 124.206 113.03) (end 124.206 81.026) (width 0.254) (layer "F.Cu") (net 5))
 (segment (start 118.11 74.93) (end 121.92 78.74) (width 0.254) (layer "B.Cu") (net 5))
 (segment (start 118.11 68.58) (end 120.65 66.04) (width 0.254) (layer "B.Cu") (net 5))
 (segment (start 118.11 68.58) (end 118.11 74.93) (width 0.254) (layer "B.Cu") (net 5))
 (segment (start 142.24 67.818) (end 142.24 68.58) (width 0.254) (layer "B.Cu") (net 5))
 (segment (start 140.462 66.04) (end 142.24 67.818) (width 0.254) (layer "B.Cu") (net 5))
 (segment (start 120.65 66.04) (end 140.462 66.04) (width 0.254) (layer "B.Cu") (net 5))
 (segment (start 149.86 68.58) (end 143.256 75.184) (width 0.254) (layer "F.Cu") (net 7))
 (segment (start 138.43 78.74) (end 137.16 78.74) (width 0.254) (layer "F.Cu") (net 7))
 (segment (start 141.986 75.184) (end 138.43 78.74) (width 0.254) (layer "F.Cu") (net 7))
 (segment (start 143.256 75.184) (end 141.986 75.184) (width 0.254) (layer "F.Cu") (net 7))
 (segment (start 142.24 88.9) (end 137.16 93.98) (width 0.254) (layer "B.Cu") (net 22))
 (segment (start 145.288 88.9) (end 142.24 88.9) (width 0.254) (layer "B.Cu") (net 22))
 (segment (start 131.318 112.522) (end 137.16 106.68) (width 0.254) (layer "F.Cu") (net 13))
 (segment (start 131.318 115.57) (end 131.318 112.522) (width 0.254) (layer "F.Cu") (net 13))
 (segment (start 137.16 90.932) (end 137.16 91.44) (width 0.254) (layer "F.Cu") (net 28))
 (segment (start 134.112 87.884) (end 137.16 90.932) (width 0.254) (layer "F.Cu") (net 28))
 (segment (start 127.254 82.296) (end 127.254 83.566) (width 0.254) (layer "B.Cu") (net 25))
 (segment (start 127.254 83.566) (end 121.92 88.9) (width 0.254) (layer "B.Cu") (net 25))
 (segment (start 125.476 91.44) (end 125.73 91.694) (width 0.254) (layer "B.Cu") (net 24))
 (segment (start 121.92 91.44) (end 125.476 91.44) (width 0.254) (layer "B.Cu") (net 24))
 (segment (start 151.13 96.52) (end 149.86 97.79) (width 0.254) (layer "F.Cu") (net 11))
 (segment (start 153.67 96.52) (end 151.13 96.52) (width 0.254) (layer "F.Cu") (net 11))
 (segment (start 153.67 93.98) (end 149.86 93.98) (width 0.254) (layer "F.Cu") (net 4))
 (segment (start 153.67 99.06) (end 152.4 99.06) (width 0.254) (layer "F.Cu") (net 10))
 (segment (start 152.4 99.06) (end 149.86 101.6) (width 0.254) (layer "F.Cu") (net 10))
 (segment (start 147.828 109.22) (end 147.828 107.442) (width 0.254) (layer "F.Cu") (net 9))
 (segment (start 147.828 107.442) (end 153.67 101.6) (width 0.254) (layer "F.Cu") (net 9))
 (segment (start 153.67 109.22) (end 153.67 104.14) (width 0.254) (layer "F.Cu") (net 2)))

